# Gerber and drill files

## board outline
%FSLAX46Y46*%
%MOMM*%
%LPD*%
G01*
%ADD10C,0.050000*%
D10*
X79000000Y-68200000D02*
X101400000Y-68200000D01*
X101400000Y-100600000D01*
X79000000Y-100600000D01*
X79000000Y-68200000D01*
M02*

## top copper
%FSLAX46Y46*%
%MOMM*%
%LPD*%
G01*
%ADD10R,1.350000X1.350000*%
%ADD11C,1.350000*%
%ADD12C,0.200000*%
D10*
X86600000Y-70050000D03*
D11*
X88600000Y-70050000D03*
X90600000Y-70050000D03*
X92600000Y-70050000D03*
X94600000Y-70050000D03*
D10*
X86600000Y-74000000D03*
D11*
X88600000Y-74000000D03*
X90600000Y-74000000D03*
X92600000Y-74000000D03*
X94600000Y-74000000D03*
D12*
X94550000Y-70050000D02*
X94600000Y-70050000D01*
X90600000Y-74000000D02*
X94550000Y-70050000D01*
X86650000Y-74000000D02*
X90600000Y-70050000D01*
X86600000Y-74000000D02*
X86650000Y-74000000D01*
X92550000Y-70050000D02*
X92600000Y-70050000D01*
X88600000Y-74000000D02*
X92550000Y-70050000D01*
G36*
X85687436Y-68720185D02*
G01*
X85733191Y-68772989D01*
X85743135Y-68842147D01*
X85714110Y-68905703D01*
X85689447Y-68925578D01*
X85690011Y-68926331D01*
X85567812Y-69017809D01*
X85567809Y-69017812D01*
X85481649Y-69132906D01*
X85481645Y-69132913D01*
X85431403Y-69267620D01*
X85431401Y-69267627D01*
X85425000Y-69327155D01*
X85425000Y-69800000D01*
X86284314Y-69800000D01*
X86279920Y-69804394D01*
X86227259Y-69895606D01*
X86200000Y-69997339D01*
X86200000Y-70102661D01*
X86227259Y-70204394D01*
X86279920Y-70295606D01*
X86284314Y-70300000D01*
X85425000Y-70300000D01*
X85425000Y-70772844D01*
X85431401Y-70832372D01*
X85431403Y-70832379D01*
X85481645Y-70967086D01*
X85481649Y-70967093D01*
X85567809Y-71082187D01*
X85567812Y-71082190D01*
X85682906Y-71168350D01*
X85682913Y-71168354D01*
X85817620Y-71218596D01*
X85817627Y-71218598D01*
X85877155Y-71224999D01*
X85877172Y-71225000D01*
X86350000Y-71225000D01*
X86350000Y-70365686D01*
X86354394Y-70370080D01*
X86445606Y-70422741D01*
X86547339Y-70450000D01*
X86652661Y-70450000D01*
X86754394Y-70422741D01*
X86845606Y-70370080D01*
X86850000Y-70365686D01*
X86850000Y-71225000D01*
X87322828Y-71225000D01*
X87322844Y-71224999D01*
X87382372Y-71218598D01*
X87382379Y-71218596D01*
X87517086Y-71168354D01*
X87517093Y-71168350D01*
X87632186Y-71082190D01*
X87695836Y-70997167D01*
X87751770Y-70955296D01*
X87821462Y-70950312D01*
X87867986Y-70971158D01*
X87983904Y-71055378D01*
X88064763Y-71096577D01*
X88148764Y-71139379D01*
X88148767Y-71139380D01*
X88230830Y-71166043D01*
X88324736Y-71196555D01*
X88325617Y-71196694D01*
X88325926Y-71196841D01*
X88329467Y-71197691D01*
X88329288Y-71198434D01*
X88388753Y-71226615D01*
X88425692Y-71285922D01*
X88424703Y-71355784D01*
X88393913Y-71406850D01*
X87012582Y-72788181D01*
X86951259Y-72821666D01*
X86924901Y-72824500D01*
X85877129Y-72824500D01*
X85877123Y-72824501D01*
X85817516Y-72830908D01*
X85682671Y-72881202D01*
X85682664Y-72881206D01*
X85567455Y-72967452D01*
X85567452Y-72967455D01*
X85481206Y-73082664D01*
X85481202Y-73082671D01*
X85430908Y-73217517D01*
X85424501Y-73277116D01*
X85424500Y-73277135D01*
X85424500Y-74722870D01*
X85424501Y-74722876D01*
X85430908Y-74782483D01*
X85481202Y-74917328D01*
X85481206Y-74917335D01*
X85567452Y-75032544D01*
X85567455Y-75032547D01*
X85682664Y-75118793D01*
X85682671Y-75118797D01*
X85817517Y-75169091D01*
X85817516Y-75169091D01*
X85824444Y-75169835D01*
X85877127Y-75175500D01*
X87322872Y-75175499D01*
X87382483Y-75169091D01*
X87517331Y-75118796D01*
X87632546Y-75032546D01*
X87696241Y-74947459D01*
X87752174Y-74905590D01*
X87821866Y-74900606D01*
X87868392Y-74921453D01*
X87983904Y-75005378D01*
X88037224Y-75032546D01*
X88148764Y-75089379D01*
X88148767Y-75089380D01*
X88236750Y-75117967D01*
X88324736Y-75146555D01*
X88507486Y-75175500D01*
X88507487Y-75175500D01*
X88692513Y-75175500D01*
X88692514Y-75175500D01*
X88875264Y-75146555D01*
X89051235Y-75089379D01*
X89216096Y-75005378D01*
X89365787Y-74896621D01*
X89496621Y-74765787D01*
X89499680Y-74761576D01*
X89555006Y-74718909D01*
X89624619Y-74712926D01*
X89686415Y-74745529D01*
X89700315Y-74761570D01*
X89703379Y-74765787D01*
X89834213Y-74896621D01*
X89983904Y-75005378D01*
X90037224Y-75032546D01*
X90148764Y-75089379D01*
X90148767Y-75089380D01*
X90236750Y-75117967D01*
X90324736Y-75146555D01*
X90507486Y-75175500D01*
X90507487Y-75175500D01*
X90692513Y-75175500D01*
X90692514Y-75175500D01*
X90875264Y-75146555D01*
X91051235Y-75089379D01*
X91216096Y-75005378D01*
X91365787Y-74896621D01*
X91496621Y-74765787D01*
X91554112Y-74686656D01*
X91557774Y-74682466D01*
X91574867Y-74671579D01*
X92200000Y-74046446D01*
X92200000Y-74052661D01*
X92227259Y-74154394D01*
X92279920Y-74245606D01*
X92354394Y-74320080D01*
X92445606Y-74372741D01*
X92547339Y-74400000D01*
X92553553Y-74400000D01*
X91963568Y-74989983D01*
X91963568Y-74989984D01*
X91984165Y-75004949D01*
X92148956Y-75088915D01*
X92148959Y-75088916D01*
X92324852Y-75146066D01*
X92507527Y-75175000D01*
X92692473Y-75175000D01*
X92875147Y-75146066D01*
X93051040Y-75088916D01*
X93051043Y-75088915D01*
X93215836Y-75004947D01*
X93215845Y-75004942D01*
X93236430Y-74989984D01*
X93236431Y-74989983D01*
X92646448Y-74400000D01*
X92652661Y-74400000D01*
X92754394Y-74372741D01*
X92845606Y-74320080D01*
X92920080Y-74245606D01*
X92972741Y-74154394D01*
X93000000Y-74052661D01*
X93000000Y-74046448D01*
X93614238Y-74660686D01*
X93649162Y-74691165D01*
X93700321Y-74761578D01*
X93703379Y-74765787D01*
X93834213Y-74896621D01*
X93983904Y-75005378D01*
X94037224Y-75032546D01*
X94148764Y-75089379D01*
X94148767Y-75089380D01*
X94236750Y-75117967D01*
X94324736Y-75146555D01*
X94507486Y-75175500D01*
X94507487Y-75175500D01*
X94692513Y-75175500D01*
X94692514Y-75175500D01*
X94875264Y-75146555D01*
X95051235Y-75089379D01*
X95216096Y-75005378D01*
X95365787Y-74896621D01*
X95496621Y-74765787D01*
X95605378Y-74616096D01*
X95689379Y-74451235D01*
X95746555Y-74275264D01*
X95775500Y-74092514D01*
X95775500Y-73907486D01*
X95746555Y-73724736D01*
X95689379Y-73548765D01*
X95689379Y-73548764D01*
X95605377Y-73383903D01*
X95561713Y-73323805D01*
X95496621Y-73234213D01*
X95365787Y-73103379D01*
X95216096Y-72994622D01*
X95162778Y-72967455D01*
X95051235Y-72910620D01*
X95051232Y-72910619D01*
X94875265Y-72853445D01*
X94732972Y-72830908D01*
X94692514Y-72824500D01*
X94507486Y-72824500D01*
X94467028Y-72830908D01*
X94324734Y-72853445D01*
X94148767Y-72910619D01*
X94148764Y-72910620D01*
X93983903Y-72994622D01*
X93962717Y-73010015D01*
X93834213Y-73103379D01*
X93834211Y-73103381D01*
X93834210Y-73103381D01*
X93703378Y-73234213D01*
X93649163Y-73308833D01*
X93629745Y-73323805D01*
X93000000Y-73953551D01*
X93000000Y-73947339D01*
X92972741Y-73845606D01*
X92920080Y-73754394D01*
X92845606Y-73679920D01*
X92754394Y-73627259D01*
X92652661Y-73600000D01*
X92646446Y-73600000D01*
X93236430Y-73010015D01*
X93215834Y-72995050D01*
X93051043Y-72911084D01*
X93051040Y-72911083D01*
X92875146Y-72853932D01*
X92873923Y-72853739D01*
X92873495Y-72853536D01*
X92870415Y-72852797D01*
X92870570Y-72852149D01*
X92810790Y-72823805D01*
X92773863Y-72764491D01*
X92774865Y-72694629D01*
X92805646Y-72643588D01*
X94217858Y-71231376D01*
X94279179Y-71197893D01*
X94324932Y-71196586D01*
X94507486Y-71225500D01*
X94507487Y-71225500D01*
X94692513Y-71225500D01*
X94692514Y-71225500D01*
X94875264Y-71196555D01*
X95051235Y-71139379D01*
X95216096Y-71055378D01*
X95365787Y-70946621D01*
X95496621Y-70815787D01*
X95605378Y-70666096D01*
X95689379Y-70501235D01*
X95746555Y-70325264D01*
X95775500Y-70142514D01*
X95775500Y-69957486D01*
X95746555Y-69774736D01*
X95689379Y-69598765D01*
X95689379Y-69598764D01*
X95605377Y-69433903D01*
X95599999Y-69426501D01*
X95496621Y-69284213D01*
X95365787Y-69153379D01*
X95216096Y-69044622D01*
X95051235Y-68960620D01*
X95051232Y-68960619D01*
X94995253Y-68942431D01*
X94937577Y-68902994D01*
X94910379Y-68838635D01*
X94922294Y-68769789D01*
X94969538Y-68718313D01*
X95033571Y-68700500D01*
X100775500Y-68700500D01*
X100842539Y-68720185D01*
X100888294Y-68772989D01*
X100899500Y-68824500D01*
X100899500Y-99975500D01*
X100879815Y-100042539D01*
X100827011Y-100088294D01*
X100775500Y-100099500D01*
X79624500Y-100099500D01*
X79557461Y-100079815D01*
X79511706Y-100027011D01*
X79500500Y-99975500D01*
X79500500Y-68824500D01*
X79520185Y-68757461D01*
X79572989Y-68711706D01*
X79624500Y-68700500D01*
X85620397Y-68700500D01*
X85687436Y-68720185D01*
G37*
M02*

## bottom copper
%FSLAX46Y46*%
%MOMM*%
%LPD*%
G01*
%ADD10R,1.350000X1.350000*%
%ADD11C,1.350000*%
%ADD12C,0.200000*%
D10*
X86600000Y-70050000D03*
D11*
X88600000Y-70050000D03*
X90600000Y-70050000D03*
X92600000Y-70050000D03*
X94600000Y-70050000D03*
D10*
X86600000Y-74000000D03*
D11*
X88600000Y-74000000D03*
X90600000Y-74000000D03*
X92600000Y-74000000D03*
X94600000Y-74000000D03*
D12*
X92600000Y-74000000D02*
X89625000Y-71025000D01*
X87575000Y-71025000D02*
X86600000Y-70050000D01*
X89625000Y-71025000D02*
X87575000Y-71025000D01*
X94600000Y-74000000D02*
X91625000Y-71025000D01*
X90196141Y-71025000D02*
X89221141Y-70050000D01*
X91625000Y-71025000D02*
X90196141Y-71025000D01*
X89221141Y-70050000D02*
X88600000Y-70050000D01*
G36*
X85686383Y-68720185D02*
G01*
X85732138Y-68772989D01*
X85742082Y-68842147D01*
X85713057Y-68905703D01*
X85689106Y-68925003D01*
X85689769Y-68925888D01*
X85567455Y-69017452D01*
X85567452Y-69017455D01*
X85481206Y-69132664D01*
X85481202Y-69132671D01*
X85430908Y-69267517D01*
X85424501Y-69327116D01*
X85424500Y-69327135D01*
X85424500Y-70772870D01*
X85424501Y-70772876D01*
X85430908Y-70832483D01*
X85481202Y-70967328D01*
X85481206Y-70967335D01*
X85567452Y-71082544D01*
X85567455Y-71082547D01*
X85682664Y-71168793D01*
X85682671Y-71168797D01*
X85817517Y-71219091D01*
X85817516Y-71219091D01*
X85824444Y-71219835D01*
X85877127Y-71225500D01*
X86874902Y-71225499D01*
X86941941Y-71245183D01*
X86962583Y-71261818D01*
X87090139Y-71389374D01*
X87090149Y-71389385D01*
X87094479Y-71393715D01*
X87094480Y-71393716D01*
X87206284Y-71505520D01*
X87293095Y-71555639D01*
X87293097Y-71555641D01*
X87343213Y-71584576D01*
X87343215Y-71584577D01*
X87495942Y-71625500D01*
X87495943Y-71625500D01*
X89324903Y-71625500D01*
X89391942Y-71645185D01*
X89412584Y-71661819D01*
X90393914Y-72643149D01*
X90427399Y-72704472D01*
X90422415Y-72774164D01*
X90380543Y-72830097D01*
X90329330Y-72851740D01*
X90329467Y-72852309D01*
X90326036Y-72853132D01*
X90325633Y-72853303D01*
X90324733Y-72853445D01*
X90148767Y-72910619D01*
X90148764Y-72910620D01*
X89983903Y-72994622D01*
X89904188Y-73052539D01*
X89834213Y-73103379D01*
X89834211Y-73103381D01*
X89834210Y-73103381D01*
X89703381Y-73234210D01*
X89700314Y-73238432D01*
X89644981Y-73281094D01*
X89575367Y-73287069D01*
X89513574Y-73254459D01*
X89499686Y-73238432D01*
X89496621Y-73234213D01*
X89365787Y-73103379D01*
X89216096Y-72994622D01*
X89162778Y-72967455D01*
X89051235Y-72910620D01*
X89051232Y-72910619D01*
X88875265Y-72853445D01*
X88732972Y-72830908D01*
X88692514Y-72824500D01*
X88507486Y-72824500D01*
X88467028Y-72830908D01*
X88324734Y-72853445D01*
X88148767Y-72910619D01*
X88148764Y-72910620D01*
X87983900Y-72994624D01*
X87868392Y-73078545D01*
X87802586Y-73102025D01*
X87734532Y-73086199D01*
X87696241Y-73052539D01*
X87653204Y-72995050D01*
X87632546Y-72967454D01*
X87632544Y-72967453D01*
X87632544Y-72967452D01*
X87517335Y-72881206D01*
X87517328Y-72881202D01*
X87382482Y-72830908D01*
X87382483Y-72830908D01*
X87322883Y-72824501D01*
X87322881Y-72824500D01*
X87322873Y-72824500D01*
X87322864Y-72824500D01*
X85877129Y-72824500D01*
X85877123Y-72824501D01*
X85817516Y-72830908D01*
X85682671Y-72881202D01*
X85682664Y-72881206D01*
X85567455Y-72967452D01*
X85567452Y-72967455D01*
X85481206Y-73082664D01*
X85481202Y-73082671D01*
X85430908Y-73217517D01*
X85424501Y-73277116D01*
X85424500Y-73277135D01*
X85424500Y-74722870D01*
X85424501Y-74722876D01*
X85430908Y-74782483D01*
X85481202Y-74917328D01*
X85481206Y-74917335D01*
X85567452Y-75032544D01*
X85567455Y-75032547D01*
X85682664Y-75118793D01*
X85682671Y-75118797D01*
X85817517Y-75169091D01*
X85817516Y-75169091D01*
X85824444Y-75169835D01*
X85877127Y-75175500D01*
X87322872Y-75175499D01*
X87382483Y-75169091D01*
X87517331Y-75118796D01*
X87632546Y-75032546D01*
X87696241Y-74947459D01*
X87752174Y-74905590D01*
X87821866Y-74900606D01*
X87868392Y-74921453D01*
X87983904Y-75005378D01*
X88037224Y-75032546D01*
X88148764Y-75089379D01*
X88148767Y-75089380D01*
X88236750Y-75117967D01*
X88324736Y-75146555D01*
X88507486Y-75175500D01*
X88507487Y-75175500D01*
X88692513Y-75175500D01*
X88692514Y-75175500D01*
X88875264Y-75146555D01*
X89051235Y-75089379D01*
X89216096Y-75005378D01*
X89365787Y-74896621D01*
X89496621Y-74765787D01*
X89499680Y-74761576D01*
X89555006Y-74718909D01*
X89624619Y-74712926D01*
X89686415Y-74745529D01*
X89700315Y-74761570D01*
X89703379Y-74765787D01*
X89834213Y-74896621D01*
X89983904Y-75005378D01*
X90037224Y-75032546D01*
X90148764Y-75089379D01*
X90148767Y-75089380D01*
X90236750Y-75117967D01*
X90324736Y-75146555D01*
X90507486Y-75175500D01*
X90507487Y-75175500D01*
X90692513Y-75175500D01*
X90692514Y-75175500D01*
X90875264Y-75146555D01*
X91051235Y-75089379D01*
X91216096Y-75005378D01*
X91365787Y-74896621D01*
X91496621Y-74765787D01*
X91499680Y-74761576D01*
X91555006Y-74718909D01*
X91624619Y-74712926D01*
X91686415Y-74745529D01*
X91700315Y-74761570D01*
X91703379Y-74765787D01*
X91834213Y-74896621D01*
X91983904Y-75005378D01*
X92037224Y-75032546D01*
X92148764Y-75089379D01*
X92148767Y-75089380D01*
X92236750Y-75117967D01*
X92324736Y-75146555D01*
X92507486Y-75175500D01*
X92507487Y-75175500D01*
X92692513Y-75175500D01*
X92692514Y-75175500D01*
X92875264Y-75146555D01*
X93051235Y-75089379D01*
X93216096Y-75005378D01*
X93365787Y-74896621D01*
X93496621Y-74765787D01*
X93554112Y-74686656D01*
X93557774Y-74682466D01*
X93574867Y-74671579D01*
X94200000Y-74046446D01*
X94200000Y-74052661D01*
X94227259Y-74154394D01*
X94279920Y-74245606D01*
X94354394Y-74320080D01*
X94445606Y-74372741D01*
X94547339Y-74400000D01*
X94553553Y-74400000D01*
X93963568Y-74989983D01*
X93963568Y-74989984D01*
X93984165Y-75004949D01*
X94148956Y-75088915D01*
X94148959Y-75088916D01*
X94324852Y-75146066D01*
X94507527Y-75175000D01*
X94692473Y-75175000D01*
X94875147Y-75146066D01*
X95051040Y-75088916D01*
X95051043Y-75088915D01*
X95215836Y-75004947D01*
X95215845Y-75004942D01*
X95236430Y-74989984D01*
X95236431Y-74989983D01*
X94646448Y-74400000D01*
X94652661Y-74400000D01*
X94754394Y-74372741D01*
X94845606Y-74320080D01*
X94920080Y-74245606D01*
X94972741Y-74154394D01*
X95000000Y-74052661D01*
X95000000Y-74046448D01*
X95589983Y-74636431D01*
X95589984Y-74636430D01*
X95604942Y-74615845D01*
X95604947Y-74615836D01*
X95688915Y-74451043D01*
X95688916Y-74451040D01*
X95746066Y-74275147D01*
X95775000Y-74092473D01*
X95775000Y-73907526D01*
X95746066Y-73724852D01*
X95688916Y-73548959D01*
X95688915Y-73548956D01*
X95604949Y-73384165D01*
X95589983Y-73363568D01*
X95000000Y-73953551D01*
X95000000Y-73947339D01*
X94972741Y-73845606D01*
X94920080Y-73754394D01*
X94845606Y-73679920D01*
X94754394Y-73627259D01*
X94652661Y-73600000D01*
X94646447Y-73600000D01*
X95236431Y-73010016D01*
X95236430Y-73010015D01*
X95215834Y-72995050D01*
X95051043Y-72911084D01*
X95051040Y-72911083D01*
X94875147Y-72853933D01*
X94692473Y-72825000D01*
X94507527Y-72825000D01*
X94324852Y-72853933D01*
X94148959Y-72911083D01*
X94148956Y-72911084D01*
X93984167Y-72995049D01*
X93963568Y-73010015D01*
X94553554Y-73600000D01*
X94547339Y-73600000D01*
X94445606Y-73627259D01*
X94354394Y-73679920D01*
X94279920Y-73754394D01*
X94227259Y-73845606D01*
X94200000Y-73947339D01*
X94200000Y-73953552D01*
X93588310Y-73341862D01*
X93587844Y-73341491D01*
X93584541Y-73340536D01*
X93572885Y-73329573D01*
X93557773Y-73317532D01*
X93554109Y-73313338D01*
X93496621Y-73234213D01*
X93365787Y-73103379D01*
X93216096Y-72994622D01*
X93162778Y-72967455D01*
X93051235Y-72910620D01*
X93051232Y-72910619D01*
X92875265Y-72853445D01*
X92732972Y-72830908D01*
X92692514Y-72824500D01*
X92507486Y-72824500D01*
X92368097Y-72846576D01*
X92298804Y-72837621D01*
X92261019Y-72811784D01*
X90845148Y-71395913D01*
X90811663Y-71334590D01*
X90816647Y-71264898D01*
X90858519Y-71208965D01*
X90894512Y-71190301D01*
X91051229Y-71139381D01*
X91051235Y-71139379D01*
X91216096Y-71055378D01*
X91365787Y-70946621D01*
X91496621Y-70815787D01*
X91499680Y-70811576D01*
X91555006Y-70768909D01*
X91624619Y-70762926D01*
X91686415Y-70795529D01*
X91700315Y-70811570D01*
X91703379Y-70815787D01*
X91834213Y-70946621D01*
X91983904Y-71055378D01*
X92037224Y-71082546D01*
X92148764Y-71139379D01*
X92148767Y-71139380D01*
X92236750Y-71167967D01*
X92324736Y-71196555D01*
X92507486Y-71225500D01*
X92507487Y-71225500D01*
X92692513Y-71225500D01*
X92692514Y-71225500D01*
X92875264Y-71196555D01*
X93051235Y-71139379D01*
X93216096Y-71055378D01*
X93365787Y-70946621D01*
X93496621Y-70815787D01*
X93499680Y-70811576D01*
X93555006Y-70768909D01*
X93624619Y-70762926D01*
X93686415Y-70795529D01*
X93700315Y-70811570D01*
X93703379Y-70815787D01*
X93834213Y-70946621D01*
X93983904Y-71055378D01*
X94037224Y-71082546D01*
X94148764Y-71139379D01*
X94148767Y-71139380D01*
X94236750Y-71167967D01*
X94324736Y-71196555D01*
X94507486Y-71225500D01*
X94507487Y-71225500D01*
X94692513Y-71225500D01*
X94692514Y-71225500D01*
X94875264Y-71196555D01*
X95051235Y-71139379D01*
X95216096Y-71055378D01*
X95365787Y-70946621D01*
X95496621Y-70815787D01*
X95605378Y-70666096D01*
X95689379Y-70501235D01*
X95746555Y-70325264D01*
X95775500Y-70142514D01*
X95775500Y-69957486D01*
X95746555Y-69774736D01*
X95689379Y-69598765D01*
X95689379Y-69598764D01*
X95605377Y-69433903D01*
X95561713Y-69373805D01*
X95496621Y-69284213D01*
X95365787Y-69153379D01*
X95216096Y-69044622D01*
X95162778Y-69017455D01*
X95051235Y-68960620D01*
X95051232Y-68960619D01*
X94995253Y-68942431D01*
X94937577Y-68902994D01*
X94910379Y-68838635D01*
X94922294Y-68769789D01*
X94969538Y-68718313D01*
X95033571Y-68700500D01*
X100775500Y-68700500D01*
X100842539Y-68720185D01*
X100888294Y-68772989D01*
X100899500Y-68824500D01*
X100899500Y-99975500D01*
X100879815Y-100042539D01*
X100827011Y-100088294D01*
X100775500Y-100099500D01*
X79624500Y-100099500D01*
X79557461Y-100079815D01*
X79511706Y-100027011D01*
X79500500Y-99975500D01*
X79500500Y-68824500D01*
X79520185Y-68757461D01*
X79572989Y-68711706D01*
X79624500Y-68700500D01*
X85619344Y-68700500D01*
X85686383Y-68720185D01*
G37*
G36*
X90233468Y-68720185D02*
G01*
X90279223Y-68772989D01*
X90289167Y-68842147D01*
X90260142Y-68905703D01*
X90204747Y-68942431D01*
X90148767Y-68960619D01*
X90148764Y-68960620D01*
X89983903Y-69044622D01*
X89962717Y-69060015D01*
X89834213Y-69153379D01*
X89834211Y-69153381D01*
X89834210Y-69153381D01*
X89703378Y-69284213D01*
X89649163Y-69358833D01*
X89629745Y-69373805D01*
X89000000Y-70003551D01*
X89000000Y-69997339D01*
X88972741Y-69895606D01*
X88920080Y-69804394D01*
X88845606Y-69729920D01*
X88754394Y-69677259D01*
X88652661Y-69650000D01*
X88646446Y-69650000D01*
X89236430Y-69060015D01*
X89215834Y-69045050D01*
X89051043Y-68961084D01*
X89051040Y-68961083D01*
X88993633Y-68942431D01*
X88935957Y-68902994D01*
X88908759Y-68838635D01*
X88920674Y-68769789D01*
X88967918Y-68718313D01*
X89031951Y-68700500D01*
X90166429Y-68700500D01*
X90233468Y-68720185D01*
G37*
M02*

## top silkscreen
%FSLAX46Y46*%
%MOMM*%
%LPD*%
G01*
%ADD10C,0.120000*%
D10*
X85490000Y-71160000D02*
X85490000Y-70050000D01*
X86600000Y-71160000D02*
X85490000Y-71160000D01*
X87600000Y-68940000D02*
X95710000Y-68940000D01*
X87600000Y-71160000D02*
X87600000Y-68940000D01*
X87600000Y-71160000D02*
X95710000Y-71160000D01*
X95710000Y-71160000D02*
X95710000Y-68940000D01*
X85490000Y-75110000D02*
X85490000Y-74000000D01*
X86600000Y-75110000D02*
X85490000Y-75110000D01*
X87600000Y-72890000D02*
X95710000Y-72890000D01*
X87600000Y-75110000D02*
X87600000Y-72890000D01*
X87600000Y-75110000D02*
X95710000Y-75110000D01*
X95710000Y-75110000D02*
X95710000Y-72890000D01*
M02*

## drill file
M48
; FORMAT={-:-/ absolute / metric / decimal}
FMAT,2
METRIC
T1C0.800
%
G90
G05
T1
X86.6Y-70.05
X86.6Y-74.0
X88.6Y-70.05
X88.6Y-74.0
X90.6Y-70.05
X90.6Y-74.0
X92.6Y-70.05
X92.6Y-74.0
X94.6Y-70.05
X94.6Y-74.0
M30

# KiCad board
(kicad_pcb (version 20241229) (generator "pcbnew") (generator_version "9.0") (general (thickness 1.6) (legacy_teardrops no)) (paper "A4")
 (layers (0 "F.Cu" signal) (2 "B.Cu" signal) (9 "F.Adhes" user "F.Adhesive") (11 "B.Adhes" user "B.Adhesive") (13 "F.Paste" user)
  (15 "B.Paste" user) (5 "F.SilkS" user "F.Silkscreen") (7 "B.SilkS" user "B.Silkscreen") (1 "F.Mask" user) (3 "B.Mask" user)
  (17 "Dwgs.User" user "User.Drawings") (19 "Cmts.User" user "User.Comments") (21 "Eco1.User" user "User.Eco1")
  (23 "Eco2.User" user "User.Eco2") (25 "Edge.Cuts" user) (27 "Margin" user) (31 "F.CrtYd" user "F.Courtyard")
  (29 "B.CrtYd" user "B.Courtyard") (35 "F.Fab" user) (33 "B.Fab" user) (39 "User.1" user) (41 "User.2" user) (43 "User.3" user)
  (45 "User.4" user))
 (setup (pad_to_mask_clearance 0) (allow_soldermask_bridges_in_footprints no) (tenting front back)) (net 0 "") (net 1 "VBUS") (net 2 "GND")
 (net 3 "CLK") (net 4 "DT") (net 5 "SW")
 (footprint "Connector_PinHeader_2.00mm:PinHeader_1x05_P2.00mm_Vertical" (layer "F.Cu") (at 86.6 70.05 90)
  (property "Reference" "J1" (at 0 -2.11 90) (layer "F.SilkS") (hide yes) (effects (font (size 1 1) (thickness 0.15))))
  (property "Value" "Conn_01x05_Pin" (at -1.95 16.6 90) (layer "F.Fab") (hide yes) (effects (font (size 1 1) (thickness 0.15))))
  (fp_line (start -1.11 -1.11) (end 0 -1.11) (stroke (width 0.12) (type solid)) (layer "F.SilkS"))
  (fp_line (start -1.11 0) (end -1.11 -1.11) (stroke (width 0.12) (type solid)) (layer "F.SilkS"))
  (fp_line (start 1.11 1) (end 1.11 9.11) (stroke (width 0.12) (type solid)) (layer "F.SilkS"))
  (fp_line (start -1.11 1) (end 1.11 1) (stroke (width 0.12) (type solid)) (layer "F.SilkS"))
  (fp_line (start -1.11 1) (end -1.11 9.11) (stroke (width 0.12) (type solid)) (layer "F.SilkS"))
  (fp_line (start -1.11 9.11) (end 1.11 9.11) (stroke (width 0.12) (type solid)) (layer "F.SilkS"))
  (pad "1" thru_hole rect (at 0 0 90) (size 1.35 1.35) (drill 0.8) (layers "*.Cu" "*.Mask") (remove_unused_layers no) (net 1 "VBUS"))
  (pad "2" thru_hole circle (at 0 2 90) (size 1.35 1.35) (drill 0.8) (layers "*.Cu" "*.Mask") (remove_unused_layers no) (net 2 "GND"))
  (pad "3" thru_hole circle (at 0 4 90) (size 1.35 1.35) (drill 0.8) (layers "*.Cu" "*.Mask") (remove_unused_layers no) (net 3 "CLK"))
  (pad "4" thru_hole circle (at 0 6 90) (size 1.35 1.35) (drill 0.8) (layers "*.Cu" "*.Mask") (remove_unused_layers no) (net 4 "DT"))
  (pad "5" thru_hole circle (at 0 8 90) (size 1.35 1.35) (drill 0.8) (layers "*.Cu" "*.Mask") (remove_unused_layers no) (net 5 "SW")))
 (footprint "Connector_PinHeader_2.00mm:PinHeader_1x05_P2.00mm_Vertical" (layer "F.Cu") (at 86.6 74 90)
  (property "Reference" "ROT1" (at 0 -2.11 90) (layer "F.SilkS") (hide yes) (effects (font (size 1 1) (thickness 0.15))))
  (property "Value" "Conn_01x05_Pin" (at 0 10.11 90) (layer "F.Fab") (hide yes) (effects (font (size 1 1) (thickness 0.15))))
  (fp_line (start -1.11 -1.11) (end 0 -1.11) (stroke (width 0.12) (type solid)) (layer "F.SilkS"))
  (fp_line (start -1.11 0) (end -1.11 -1.11) (stroke (width 0.12) (type solid)) (layer "F.SilkS"))
  (fp_line (start 1.11 1) (end 1.11 9.11) (stroke (width 0.12) (type solid)) (layer "F.SilkS"))
  (fp_line (start -1.11 1) (end 1.11 1) (stroke (width 0.12) (type solid)) (layer "F.SilkS"))
  (fp_line (start -1.11 1) (end -1.11 9.11) (stroke (width 0.12) (type solid)) (layer "F.SilkS"))
  (fp_line (start -1.11 9.11) (end 1.11 9.11) (stroke (width 0.12) (type solid)) (layer "F.SilkS"))
  (pad "1" thru_hole rect (at 0 0 90) (size 1.35 1.35) (drill 0.8) (layers "*.Cu" "*.Mask") (remove_unused_layers no) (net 3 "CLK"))
  (pad "2" thru_hole circle (at 0 2 90) (size 1.35 1.35) (drill 0.8) (layers "*.Cu" "*.Mask") (remove_unused_layers no) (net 4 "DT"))
  (pad "3" thru_hole circle (at 0 4 90) (size 1.35 1.35) (drill 0.8) (layers "*.Cu" "*.Mask") (remove_unused_layers no) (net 5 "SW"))
  (pad "4" thru_hole circle (at 0 6 90) (size 1.35 1.35) (drill 0.8) (layers "*.Cu" "*.Mask") (remove_unused_layers no) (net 1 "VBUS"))
  (pad "5" thru_hole circle (at 0 8 90) (size 1.35 1.35) (drill 0.8) (layers "*.Cu" "*.Mask") (remove_unused_layers no) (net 2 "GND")))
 (gr_rect (start 79 68.2) (end 101.4 100.6) (stroke (width 0.05) (type default)) (fill no) (layer "Edge.Cuts"))
 (segment (start 94.55 70.05) (end 94.6 70.05) (width 0.2) (layer "F.Cu") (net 5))
 (segment (start 90.6 74) (end 94.55 70.05) (width 0.2) (layer "F.Cu") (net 5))
 (segment (start 86.65 74) (end 90.6 70.05) (width 0.2) (layer "F.Cu") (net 3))
 (segment (start 86.6 74) (end 86.65 74) (width 0.2) (layer "F.Cu") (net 3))
 (segment (start 92.6 74) (end 89.625 71.025) (width 0.2) (layer "B.Cu") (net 1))
 (segment (start 87.575 71.025) (end 86.6 70.05) (width 0.2) (layer "B.Cu") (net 1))
 (segment (start 89.625 71.025) (end 87.575 71.025) (width 0.2) (layer "B.Cu") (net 1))
 (segment (start 92.55 70.05) (end 92.6 70.05) (width 0.2) (layer "F.Cu") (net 4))
 (segment (start 88.6 74) (end 92.55 70.05) (width 0.2) (layer "F.Cu") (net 4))
 (segment (start 94.6 74) (end 91.625 71.025) (width 0.2) (layer "B.Cu") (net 2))
 (segment (start 90.196141 71.025) (end 89.221141 70.05) (width 0.2) (layer "B.Cu") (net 2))
 (segment (start 91.625 71.025) (end 90.196141 71.025) (width 0.2) (layer "B.Cu") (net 2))
 (segment (start 89.221141 70.05) (end 88.6 70.05) (width 0.2) (layer "B.Cu") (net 2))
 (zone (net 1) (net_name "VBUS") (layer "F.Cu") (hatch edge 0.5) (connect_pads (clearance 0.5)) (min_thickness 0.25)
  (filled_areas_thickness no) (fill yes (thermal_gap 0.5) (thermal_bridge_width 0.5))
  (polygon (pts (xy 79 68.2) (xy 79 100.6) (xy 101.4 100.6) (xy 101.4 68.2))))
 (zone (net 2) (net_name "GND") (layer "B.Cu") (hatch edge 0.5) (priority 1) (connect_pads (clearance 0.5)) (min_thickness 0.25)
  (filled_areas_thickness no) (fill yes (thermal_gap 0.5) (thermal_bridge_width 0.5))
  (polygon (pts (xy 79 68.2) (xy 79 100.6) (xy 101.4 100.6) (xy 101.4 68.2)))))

